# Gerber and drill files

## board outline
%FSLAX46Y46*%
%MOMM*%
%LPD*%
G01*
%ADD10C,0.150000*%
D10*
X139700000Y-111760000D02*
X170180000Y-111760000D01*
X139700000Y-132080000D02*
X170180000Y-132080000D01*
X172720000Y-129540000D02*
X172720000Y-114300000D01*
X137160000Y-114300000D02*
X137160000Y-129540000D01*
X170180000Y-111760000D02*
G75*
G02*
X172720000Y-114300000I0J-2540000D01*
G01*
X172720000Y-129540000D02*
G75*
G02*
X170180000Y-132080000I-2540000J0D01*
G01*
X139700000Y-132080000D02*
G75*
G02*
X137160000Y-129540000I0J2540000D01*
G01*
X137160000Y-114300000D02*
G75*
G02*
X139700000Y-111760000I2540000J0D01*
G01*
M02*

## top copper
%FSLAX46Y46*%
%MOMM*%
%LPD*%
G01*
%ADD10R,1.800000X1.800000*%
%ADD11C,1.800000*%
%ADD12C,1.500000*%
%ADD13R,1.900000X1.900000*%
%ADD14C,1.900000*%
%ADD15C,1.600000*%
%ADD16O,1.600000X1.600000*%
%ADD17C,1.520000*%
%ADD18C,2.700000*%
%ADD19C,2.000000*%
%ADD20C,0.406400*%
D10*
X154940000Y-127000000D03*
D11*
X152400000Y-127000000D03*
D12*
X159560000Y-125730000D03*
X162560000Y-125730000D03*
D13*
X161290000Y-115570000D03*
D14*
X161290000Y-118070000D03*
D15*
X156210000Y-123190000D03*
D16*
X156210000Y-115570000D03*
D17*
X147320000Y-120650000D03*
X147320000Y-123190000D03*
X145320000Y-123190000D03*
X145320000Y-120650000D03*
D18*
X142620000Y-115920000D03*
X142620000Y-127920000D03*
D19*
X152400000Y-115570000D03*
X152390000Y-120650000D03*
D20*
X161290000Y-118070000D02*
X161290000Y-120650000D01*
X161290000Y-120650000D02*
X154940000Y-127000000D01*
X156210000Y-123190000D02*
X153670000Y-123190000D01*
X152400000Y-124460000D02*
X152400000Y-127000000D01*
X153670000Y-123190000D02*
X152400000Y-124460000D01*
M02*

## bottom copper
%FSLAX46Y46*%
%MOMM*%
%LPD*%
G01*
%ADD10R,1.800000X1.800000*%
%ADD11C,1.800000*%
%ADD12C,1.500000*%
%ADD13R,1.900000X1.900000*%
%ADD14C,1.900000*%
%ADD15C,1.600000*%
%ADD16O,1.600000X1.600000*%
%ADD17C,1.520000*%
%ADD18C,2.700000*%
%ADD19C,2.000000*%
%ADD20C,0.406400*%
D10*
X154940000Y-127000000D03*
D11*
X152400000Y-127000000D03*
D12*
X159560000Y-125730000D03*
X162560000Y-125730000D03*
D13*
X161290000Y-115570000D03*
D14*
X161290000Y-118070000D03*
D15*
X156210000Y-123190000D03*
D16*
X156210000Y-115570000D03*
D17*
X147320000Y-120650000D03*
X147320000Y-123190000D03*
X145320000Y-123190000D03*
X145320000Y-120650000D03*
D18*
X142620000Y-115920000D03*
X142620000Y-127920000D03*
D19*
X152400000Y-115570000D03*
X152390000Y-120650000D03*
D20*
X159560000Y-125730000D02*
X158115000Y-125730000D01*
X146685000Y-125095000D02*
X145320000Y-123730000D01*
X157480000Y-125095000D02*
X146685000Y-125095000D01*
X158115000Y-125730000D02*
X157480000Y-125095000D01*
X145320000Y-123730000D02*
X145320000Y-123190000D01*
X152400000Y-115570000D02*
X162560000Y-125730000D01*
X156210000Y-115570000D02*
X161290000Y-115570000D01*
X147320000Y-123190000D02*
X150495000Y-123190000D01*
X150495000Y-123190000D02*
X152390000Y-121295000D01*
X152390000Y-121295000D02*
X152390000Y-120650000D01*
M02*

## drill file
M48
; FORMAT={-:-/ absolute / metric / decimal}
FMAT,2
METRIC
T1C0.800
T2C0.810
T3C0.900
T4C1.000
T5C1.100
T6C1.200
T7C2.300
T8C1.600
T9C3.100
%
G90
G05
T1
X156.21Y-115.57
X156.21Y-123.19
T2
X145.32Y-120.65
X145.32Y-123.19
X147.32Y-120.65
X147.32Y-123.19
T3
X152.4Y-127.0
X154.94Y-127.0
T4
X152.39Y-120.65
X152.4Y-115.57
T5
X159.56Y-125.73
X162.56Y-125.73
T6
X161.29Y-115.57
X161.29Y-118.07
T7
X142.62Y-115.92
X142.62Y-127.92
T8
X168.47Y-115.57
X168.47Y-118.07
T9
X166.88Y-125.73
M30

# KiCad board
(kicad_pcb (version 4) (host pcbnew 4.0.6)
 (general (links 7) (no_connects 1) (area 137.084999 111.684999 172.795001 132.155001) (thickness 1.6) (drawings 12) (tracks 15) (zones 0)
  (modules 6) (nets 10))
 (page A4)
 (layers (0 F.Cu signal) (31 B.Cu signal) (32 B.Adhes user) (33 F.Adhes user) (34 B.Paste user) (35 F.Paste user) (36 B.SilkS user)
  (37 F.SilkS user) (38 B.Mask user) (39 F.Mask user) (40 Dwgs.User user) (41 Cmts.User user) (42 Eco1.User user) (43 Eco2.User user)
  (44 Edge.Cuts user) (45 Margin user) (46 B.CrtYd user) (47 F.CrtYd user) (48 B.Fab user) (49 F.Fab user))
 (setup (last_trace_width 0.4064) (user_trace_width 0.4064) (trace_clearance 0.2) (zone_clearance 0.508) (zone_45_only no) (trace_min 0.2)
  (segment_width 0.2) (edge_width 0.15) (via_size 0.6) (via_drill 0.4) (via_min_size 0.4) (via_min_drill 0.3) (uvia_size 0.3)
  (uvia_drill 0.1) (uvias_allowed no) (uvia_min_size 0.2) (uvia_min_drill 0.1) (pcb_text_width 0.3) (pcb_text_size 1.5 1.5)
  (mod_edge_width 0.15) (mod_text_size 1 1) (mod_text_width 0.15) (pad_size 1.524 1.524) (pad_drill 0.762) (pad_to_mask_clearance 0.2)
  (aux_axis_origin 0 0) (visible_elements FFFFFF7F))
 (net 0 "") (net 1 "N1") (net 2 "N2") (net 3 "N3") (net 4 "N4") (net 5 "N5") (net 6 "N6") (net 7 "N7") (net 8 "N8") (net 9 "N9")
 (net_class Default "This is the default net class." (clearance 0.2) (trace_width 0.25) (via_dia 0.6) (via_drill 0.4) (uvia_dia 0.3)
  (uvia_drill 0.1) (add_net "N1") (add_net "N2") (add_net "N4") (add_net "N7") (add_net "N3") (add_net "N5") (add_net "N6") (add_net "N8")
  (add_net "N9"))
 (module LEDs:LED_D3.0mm (layer F.Cu) (at 154.94 127 180)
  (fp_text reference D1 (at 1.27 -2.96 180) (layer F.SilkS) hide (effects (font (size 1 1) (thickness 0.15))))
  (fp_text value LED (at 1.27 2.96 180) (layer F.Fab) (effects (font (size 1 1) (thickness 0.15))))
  (pad 1 thru_hole rect (at 0 0 180) (size 1.8 1.8) (drill 0.9) (layers *.Cu *.Mask) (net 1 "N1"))
  (pad 2 thru_hole circle (at 2.54 0 180) (size 1.8 1.8) (drill 0.9) (layers *.Cu *.Mask) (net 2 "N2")))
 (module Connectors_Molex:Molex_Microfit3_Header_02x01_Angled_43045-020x (layer F.Cu) (at 162.56 125.73 90)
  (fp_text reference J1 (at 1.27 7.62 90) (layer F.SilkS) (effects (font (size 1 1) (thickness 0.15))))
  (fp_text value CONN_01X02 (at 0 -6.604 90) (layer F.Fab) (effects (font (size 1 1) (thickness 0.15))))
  (pad 2 thru_hole circle (at 0 -3 90) (size 1.5 1.5) (drill 1.1) (layers *.Cu *.Mask) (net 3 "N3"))
  (pad 1 thru_hole circle (at 0 0 90) (size 1.5 1.5) (drill 1.1) (layers *.Cu *.Mask) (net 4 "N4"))
  (pad "" np_thru_hole circle (at 0 4.32 90) (size 3.1 3.1) (drill 3.1) (layers *.Cu *.Mask)))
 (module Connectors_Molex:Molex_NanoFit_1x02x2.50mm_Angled (layer F.Cu) (at 161.29 115.57 270)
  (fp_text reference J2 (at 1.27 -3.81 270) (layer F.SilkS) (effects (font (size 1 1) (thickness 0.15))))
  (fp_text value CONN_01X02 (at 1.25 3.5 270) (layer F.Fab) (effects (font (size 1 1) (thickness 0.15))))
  (pad 1 thru_hole rect (at 0 0 270) (size 1.9 1.9) (drill 1.2) (layers *.Cu *.Mask) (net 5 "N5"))
  (pad 2 thru_hole circle (at 2.5 0 270) (size 1.9 1.9) (drill 1.2) (layers *.Cu *.Mask) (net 1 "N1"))
  (pad "" np_thru_hole circle (at 0 -7.18 270) (size 1.6 1.6) (drill 1.6) (layers *.Cu *.Mask))
  (pad "" np_thru_hole circle (at 2.5 -7.18 270) (size 1.6 1.6) (drill 1.6) (layers *.Cu *.Mask)))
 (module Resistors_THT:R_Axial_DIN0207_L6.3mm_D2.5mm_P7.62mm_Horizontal (layer F.Cu) (at 156.21 123.19 90)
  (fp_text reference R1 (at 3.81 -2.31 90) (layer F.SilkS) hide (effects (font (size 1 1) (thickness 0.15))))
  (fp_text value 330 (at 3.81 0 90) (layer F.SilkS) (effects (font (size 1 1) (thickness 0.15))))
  (pad 1 thru_hole circle (at 0 0 90) (size 1.6 1.6) (drill 0.8) (layers *.Cu *.Mask) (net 2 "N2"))
  (pad 2 thru_hole oval (at 7.62 0 90) (size 1.6 1.6) (drill 0.8) (layers *.Cu *.Mask) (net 5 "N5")))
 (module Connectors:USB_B (layer F.Cu) (at 147.32 123.19 180)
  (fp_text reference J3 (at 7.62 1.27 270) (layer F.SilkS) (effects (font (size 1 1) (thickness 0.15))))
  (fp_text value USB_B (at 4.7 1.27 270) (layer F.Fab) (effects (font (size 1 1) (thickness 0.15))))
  (pad 2 thru_hole circle (at 0 2.54 90) (size 1.52 1.52) (drill 0.81) (layers *.Cu *.Mask) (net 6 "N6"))
  (pad 1 thru_hole circle (at 0 0 90) (size 1.52 1.52) (drill 0.81) (layers *.Cu *.Mask) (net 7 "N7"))
  (pad 4 thru_hole circle (at 2 0 90) (size 1.52 1.52) (drill 0.81) (layers *.Cu *.Mask) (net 3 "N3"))
  (pad 3 thru_hole circle (at 2 2.54 90) (size 1.52 1.52) (drill 0.81) (layers *.Cu *.Mask) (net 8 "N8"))
  (pad 5 thru_hole circle (at 4.7 7.27 90) (size 2.7 2.7) (drill 2.3) (layers *.Cu *.Mask) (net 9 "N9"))
  (pad 5 thru_hole circle (at 4.7 -4.73 90) (size 2.7 2.7) (drill 2.3) (layers *.Cu *.Mask) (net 9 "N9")))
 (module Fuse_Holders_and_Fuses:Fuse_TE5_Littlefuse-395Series (layer F.Cu) (at 152.4 115.57 270)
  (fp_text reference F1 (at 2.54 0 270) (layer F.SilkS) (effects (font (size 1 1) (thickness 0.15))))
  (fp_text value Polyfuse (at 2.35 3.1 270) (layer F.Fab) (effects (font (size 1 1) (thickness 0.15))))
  (pad 1 thru_hole circle (at 0 0 270) (size 2 2) (drill 1) (layers *.Cu *.Mask) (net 4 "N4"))
  (pad 2 thru_hole circle (at 5.08 0.01 270) (size 2 2) (drill 1) (layers *.Cu *.Mask) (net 7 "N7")))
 (gr_line (start 139.7 111.76) (end 170.18 111.76) (angle 90) (layer Edge.Cuts) (width 0.15))
 (gr_line (start 139.7 132.08) (end 170.18 132.08) (angle 90) (layer Edge.Cuts) (width 0.15))
 (gr_line (start 172.72 129.54) (end 172.72 114.3) (angle 90) (layer Edge.Cuts) (width 0.15))
 (gr_line (start 137.16 114.3) (end 137.16 129.54) (angle 90) (layer Edge.Cuts) (width 0.15))
 (gr_arc (start 170.18 114.3) (end 170.18 111.76) (angle 90) (layer Edge.Cuts) (width 0.15))
 (gr_arc (start 170.18 129.54) (end 172.72 129.54) (angle 90) (layer Edge.Cuts) (width 0.15))
 (gr_arc (start 139.7 129.54) (end 139.7 132.08) (angle 90) (layer Edge.Cuts) (width 0.15))
 (gr_arc (start 139.7 114.3) (end 137.16 114.3) (angle 90) (layer Edge.Cuts) (width 0.15))
 (segment (start 161.29 118.07) (end 161.29 120.65) (width 0.4064) (layer F.Cu) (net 1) (status 400000))
 (segment (start 161.29 120.65) (end 154.94 127) (width 0.4064) (layer F.Cu) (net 1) (status 800000))
 (segment (start 156.21 123.19) (end 153.67 123.19) (width 0.4064) (layer F.Cu) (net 2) (status 400000))
 (segment (start 152.4 124.46) (end 152.4 127) (width 0.4064) (layer F.Cu) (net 2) (status 800000))
 (segment (start 153.67 123.19) (end 152.4 124.46) (width 0.4064) (layer F.Cu) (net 2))
 (segment (start 159.56 125.73) (end 158.115 125.73) (width 0.4064) (layer B.Cu) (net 3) (status 400000))
 (segment (start 146.685 125.095) (end 145.32 123.73) (width 0.4064) (layer B.Cu) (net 3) (status 800000))
 (segment (start 157.48 125.095) (end 146.685 125.095) (width 0.4064) (layer B.Cu) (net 3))
 (segment (start 158.115 125.73) (end 157.48 125.095) (width 0.4064) (layer B.Cu) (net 3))
 (segment (start 145.32 123.73) (end 145.32 123.19) (width 0.4064) (layer B.Cu) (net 3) (status C00000))
 (segment (start 152.4 115.57) (end 162.56 125.73) (width 0.4064) (layer B.Cu) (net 4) (status C00000))
 (segment (start 156.21 115.57) (end 161.29 115.57) (width 0.4064) (layer B.Cu) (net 5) (status C00000))
 (segment (start 147.32 123.19) (end 150.495 123.19) (width 0.4064) (layer B.Cu) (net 7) (status 400000))
 (segment (start 150.495 123.19) (end 152.39 121.295) (width 0.4064) (layer B.Cu) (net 7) (status 800000))
 (segment (start 152.39 121.295) (end 152.39 120.65) (width 0.4064) (layer B.Cu) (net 7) (status C00000)))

